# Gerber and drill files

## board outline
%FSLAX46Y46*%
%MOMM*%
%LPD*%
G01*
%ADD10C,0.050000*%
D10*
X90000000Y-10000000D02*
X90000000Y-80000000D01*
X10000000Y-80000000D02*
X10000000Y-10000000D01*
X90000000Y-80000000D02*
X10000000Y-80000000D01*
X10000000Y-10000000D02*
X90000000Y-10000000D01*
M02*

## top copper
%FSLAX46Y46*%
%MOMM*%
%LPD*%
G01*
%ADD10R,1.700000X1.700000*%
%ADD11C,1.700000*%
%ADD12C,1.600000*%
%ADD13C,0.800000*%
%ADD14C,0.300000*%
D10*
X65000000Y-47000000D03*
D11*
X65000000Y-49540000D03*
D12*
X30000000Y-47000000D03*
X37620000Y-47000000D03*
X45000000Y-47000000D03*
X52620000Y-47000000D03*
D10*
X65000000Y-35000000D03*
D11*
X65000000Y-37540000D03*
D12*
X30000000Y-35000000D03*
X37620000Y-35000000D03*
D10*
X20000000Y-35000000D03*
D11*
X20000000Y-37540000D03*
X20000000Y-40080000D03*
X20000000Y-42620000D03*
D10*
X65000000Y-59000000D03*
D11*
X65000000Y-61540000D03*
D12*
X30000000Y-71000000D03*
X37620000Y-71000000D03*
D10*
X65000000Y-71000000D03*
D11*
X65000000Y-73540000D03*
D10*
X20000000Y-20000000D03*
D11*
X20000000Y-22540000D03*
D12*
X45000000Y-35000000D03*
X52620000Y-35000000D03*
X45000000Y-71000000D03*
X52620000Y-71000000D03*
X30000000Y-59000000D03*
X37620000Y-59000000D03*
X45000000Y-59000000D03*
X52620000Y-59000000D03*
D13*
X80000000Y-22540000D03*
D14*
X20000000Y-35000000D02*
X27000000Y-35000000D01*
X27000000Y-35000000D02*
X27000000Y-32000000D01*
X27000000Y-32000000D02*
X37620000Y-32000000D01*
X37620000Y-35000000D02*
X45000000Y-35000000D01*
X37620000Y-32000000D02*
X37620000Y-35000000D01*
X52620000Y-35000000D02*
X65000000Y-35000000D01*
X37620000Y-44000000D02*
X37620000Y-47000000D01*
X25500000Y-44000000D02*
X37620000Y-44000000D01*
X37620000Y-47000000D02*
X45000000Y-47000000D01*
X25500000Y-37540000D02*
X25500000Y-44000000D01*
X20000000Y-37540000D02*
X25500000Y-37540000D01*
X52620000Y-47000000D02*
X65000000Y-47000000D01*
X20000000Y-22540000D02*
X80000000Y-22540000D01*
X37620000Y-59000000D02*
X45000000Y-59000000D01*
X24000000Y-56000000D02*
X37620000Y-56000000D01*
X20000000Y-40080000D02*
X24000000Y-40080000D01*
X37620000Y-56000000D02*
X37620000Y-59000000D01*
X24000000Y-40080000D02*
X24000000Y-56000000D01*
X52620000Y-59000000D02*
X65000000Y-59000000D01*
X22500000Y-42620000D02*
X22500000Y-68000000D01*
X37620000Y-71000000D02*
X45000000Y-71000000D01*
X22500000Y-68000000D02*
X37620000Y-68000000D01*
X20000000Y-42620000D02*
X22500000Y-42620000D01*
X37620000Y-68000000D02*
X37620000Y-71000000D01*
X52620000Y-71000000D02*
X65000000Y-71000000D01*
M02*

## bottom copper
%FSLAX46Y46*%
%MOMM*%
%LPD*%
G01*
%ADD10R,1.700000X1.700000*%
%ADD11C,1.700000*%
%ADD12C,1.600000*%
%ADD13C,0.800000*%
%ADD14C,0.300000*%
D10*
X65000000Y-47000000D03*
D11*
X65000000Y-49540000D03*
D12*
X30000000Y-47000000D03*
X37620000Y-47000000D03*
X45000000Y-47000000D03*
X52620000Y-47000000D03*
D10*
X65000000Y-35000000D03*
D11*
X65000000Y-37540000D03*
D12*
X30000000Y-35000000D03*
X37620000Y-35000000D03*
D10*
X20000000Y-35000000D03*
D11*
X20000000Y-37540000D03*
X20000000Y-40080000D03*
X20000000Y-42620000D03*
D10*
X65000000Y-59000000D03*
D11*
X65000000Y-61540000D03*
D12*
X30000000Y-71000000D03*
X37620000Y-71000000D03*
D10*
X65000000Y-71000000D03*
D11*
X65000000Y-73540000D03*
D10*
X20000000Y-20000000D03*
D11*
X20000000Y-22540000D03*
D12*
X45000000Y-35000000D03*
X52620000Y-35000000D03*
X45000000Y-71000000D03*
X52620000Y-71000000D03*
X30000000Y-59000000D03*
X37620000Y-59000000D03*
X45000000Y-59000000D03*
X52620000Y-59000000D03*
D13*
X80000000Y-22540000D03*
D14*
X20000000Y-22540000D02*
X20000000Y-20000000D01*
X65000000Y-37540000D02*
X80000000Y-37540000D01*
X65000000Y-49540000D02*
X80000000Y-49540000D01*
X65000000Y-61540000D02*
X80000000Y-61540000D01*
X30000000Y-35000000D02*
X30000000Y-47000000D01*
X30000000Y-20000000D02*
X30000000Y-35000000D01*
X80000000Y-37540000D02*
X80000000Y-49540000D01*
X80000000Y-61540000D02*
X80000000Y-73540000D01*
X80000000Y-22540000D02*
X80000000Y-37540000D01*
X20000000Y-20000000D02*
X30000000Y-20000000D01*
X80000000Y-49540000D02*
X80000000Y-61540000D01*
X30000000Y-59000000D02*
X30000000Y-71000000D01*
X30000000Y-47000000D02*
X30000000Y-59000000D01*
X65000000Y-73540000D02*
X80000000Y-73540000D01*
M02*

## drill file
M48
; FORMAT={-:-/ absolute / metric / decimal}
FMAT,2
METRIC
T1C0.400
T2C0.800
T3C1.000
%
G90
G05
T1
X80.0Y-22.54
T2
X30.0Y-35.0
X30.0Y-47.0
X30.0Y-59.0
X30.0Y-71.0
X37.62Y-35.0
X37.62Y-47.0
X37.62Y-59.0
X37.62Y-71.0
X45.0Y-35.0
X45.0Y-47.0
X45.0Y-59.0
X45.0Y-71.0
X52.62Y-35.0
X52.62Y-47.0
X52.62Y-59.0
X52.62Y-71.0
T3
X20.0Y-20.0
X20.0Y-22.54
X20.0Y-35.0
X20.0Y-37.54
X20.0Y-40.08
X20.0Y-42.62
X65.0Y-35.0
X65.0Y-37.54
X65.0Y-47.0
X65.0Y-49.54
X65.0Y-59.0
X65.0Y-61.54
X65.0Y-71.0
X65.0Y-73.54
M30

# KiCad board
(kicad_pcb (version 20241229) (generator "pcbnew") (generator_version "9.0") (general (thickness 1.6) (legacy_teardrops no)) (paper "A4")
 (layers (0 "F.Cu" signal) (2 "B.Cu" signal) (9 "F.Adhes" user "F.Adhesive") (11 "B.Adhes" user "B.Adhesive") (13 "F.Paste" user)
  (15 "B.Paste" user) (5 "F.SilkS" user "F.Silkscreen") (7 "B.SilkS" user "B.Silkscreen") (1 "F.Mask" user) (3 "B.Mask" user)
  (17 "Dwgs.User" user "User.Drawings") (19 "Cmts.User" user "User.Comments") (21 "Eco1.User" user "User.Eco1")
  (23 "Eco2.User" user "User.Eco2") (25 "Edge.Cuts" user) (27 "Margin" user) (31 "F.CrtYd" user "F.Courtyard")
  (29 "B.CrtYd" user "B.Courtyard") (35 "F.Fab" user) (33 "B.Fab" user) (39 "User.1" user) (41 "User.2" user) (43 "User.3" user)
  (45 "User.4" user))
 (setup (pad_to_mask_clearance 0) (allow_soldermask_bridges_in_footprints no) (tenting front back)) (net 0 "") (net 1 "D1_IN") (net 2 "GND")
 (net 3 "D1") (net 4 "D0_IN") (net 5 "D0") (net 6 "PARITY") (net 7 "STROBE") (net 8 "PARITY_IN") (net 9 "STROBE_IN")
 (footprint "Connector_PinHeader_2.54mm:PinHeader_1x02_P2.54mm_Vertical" (layer "F.Cu") (at 65 47)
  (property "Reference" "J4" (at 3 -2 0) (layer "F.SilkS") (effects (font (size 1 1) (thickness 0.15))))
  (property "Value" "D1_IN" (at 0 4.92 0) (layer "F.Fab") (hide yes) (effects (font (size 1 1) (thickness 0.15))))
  (pad "1" thru_hole rect (at 0 0) (size 1.7 1.7) (drill 1) (layers "*.Cu" "*.Mask") (remove_unused_layers no) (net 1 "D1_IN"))
  (pad "2" thru_hole circle (at 0 2.54) (size 1.7 1.7) (drill 1) (layers "*.Cu" "*.Mask") (remove_unused_layers no) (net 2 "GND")))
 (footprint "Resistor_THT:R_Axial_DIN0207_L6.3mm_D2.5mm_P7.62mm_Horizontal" (layer "F.Cu") (at 30 47)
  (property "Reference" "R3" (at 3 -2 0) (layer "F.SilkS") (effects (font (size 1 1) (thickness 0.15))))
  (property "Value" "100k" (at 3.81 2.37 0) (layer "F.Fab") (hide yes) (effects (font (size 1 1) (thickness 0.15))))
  (pad "1" thru_hole circle (at 0 0) (size 1.6 1.6) (drill 0.8) (layers "*.Cu" "*.Mask") (remove_unused_layers no) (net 2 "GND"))
  (pad "2" thru_hole circle (at 7.62 0) (size 1.6 1.6) (drill 0.8) (layers "*.Cu" "*.Mask") (remove_unused_layers no) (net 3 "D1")))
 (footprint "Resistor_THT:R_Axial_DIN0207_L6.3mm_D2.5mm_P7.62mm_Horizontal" (layer "F.Cu") (at 45 47)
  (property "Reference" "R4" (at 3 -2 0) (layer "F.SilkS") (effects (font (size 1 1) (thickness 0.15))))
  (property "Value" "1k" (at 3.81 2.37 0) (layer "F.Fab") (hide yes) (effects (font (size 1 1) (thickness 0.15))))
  (pad "1" thru_hole circle (at 0 0) (size 1.6 1.6) (drill 0.8) (layers "*.Cu" "*.Mask") (remove_unused_layers no) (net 3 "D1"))
  (pad "2" thru_hole circle (at 7.62 0) (size 1.6 1.6) (drill 0.8) (layers "*.Cu" "*.Mask") (remove_unused_layers no) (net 1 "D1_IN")))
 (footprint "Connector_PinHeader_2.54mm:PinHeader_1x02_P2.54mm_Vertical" (layer "F.Cu") (at 65 35)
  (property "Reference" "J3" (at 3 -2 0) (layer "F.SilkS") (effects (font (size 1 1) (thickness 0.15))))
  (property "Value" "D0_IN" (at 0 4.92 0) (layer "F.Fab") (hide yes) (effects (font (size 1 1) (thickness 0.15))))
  (pad "1" thru_hole rect (at 0 0) (size 1.7 1.7) (drill 1) (layers "*.Cu" "*.Mask") (remove_unused_layers no) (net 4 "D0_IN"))
  (pad "2" thru_hole circle (at 0 2.54) (size 1.7 1.7) (drill 1) (layers "*.Cu" "*.Mask") (remove_unused_layers no) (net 2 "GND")))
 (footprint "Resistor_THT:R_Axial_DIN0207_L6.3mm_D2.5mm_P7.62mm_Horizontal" (layer "F.Cu") (at 30 35)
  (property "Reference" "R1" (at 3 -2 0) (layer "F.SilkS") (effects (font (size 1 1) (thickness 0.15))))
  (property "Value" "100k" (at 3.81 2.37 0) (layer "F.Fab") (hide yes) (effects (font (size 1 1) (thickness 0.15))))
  (pad "1" thru_hole circle (at 0 0) (size 1.6 1.6) (drill 0.8) (layers "*.Cu" "*.Mask") (remove_unused_layers no) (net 2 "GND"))
  (pad "2" thru_hole circle (at 7.62 0) (size 1.6 1.6) (drill 0.8) (layers "*.Cu" "*.Mask") (remove_unused_layers no) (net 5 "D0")))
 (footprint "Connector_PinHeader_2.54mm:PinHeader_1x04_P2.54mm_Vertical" (layer "F.Cu") (at 20 35)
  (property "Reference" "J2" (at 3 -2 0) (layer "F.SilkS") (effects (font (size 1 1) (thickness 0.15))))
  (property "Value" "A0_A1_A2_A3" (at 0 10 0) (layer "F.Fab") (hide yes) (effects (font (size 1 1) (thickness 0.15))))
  (pad "1" thru_hole rect (at 0 0) (size 1.7 1.7) (drill 1) (layers "*.Cu" "*.Mask") (remove_unused_layers no) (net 5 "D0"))
  (pad "2" thru_hole circle (at 0 2.54) (size 1.7 1.7) (drill 1) (layers "*.Cu" "*.Mask") (remove_unused_layers no) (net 3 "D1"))
  (pad "3" thru_hole circle (at 0 5.08) (size 1.7 1.7) (drill 1) (layers "*.Cu" "*.Mask") (remove_unused_layers no) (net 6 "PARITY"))
  (pad "4" thru_hole circle (at 0 7.62) (size 1.7 1.7) (drill 1) (layers "*.Cu" "*.Mask") (remove_unused_layers no) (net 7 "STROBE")))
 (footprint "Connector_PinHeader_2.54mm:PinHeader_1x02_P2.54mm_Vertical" (layer "F.Cu") (at 65 59)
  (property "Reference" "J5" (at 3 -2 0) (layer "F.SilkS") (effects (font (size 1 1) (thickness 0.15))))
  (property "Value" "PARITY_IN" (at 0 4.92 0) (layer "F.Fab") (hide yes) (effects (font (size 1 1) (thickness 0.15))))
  (pad "1" thru_hole rect (at 0 0) (size 1.7 1.7) (drill 1) (layers "*.Cu" "*.Mask") (remove_unused_layers no) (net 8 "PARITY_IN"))
  (pad "2" thru_hole circle (at 0 2.54) (size 1.7 1.7) (drill 1) (layers "*.Cu" "*.Mask") (remove_unused_layers no) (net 2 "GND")))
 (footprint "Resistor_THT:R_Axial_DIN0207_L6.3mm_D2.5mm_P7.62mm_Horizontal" (layer "F.Cu") (at 30 71)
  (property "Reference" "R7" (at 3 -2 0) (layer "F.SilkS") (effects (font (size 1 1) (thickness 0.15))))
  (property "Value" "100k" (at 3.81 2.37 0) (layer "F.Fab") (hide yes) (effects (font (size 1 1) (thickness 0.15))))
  (pad "1" thru_hole circle (at 0 0) (size 1.6 1.6) (drill 0.8) (layers "*.Cu" "*.Mask") (remove_unused_layers no) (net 2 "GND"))
  (pad "2" thru_hole circle (at 7.62 0) (size 1.6 1.6) (drill 0.8) (layers "*.Cu" "*.Mask") (remove_unused_layers no) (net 7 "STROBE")))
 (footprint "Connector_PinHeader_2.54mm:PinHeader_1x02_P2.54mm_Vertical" (layer "F.Cu") (at 65 71)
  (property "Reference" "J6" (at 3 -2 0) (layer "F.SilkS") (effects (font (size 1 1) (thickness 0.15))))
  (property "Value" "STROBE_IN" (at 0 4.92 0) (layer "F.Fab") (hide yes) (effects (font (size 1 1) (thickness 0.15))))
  (pad "1" thru_hole rect (at 0 0) (size 1.7 1.7) (drill 1) (layers "*.Cu" "*.Mask") (remove_unused_layers no) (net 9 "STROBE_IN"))
  (pad "2" thru_hole circle (at 0 2.54) (size 1.7 1.7) (drill 1) (layers "*.Cu" "*.Mask") (remove_unused_layers no) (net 2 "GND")))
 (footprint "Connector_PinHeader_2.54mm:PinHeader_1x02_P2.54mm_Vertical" (layer "F.Cu") (at 20 20)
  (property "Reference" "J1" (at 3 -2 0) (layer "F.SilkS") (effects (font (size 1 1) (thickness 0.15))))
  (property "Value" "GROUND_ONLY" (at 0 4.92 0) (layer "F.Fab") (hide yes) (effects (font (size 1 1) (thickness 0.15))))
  (pad "1" thru_hole rect (at 0 0) (size 1.7 1.7) (drill 1) (layers "*.Cu" "*.Mask") (remove_unused_layers no) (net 2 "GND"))
  (pad "2" thru_hole circle (at 0 2.54) (size 1.7 1.7) (drill 1) (layers "*.Cu" "*.Mask") (remove_unused_layers no) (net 2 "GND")))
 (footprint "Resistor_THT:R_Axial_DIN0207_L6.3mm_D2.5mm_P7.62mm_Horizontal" (layer "F.Cu") (at 45 35)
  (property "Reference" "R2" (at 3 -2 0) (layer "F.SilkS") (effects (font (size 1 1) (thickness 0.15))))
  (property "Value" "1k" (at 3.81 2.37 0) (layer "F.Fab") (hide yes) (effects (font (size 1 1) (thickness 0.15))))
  (pad "1" thru_hole circle (at 0 0) (size 1.6 1.6) (drill 0.8) (layers "*.Cu" "*.Mask") (remove_unused_layers no) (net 5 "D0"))
  (pad "2" thru_hole circle (at 7.62 0) (size 1.6 1.6) (drill 0.8) (layers "*.Cu" "*.Mask") (remove_unused_layers no) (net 4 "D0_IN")))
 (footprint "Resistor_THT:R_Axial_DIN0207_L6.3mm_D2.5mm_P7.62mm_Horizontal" (layer "F.Cu") (at 45 71)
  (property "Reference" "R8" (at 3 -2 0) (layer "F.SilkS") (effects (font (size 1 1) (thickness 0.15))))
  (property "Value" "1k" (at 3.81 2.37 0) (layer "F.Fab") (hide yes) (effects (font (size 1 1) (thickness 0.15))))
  (pad "1" thru_hole circle (at 0 0) (size 1.6 1.6) (drill 0.8) (layers "*.Cu" "*.Mask") (remove_unused_layers no) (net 7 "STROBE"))
  (pad "2" thru_hole circle (at 7.62 0) (size 1.6 1.6) (drill 0.8) (layers "*.Cu" "*.Mask") (remove_unused_layers no) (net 9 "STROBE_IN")))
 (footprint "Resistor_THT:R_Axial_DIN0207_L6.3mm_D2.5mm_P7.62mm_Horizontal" (layer "F.Cu") (at 30 59)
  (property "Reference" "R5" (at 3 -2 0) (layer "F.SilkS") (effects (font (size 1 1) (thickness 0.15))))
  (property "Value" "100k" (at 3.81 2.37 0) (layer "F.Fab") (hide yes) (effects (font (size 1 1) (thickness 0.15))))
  (pad "1" thru_hole circle (at 0 0) (size 1.6 1.6) (drill 0.8) (layers "*.Cu" "*.Mask") (remove_unused_layers no) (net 2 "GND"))
  (pad "2" thru_hole circle (at 7.62 0) (size 1.6 1.6) (drill 0.8) (layers "*.Cu" "*.Mask") (remove_unused_layers no) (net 6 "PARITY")))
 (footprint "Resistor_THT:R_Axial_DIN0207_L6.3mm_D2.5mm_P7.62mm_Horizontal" (layer "F.Cu") (at 45 59)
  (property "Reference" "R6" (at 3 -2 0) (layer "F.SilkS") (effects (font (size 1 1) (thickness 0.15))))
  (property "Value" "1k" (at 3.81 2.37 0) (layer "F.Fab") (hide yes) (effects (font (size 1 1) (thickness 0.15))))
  (pad "1" thru_hole circle (at 0 0) (size 1.6 1.6) (drill 0.8) (layers "*.Cu" "*.Mask") (remove_unused_layers no) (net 6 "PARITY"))
  (pad "2" thru_hole circle (at 7.62 0) (size 1.6 1.6) (drill 0.8) (layers "*.Cu" "*.Mask") (remove_unused_layers no) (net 8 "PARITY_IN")))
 (gr_line (start 90 10) (end 90 80) (stroke (width 0.05) (type default)) (layer "Edge.Cuts"))
 (gr_line (start 10 80) (end 10 10) (stroke (width 0.05) (type default)) (layer "Edge.Cuts"))
 (gr_line (start 90 80) (end 10 80) (stroke (width 0.05) (type default)) (layer "Edge.Cuts"))
 (gr_line (start 10 10) (end 90 10) (stroke (width 0.05) (type default)) (layer "Edge.Cuts"))
 (segment (start 20 35) (end 27 35) (width 0.3) (layer "F.Cu") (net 5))
 (segment (start 27 35) (end 27 32) (width 0.3) (layer "F.Cu") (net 5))
 (segment (start 27 32) (end 37.62 32) (width 0.3) (layer "F.Cu") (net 5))
 (segment (start 37.62 35) (end 45 35) (width 0.3) (layer "F.Cu") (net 5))
 (segment (start 37.62 32) (end 37.62 35) (width 0.3) (layer "F.Cu") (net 5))
 (segment (start 52.62 35) (end 65 35) (width 0.3) (layer "F.Cu") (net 4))
 (segment (start 37.62 44) (end 37.62 47) (width 0.3) (layer "F.Cu") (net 3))
 (segment (start 25.5 44) (end 37.62 44) (width 0.3) (layer "F.Cu") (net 3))
 (segment (start 37.62 47) (end 45 47) (width 0.3) (layer "F.Cu") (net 3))
 (segment (start 25.5 37.54) (end 25.5 44) (width 0.3) (layer "F.Cu") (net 3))
 (segment (start 20 37.54) (end 25.5 37.54) (width 0.3) (layer "F.Cu") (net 3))
 (segment (start 52.62 47) (end 65 47) (width 0.3) (layer "F.Cu") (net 1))
 (segment (start 20 22.54) (end 80 22.54) (width 0.3) (layer "F.Cu") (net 2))
 (via (at 80 22.54) (size 0.8) (drill 0.4) (layers "F.Cu" "B.Cu") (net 2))
 (segment (start 20 22.54) (end 20 20) (width 0.3) (layer "B.Cu") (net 2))
 (segment (start 65 37.54) (end 80 37.54) (width 0.3) (layer "B.Cu") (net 2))
 (segment (start 65 49.54) (end 80 49.54) (width 0.3) (layer "B.Cu") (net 2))
 (segment (start 65 61.54) (end 80 61.54) (width 0.3) (layer "B.Cu") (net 2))
 (segment (start 30 35) (end 30 47) (width 0.3) (layer "B.Cu") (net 2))
 (segment (start 30 20) (end 30 35) (width 0.3) (layer "B.Cu") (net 2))
 (segment (start 80 37.54) (end 80 49.54) (width 0.3) (layer "B.Cu") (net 2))
 (segment (start 80 61.54) (end 80 73.54) (width 0.3) (layer "B.Cu") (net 2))
 (segment (start 80 22.54) (end 80 37.54) (width 0.3) (layer "B.Cu") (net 2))
 (segment (start 20 20) (end 30 20) (width 0.3) (layer "B.Cu") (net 2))
 (segment (start 80 49.54) (end 80 61.54) (width 0.3) (layer "B.Cu") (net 2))
 (segment (start 30 59) (end 30 71) (width 0.3) (layer "B.Cu") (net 2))
 (segment (start 30 47) (end 30 59) (width 0.3) (layer "B.Cu") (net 2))
 (segment (start 65 73.54) (end 80 73.54) (width 0.3) (layer "B.Cu") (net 2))
 (segment (start 37.62 59) (end 45 59) (width 0.3) (layer "F.Cu") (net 6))
 (segment (start 24 56) (end 37.62 56) (width 0.3) (layer "F.Cu") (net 6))
 (segment (start 20 40.08) (end 24 40.08) (width 0.3) (layer "F.Cu") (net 6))
 (segment (start 37.62 56) (end 37.62 59) (width 0.3) (layer "F.Cu") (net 6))
 (segment (start 24 40.08) (end 24 56) (width 0.3) (layer "F.Cu") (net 6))
 (segment (start 52.62 59) (end 65 59) (width 0.3) (layer "F.Cu") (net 8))
 (segment (start 22.5 42.62) (end 22.5 68) (width 0.3) (layer "F.Cu") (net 7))
 (segment (start 37.62 71) (end 45 71) (width 0.3) (layer "F.Cu") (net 7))
 (segment (start 22.5 68) (end 37.62 68) (width 0.3) (layer "F.Cu") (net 7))
 (segment (start 20 42.62) (end 22.5 42.62) (width 0.3) (layer "F.Cu") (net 7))
 (segment (start 37.62 68) (end 37.62 71) (width 0.3) (layer "F.Cu") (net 7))
 (segment (start 52.62 71) (end 65 71) (width 0.3) (layer "F.Cu") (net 9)))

